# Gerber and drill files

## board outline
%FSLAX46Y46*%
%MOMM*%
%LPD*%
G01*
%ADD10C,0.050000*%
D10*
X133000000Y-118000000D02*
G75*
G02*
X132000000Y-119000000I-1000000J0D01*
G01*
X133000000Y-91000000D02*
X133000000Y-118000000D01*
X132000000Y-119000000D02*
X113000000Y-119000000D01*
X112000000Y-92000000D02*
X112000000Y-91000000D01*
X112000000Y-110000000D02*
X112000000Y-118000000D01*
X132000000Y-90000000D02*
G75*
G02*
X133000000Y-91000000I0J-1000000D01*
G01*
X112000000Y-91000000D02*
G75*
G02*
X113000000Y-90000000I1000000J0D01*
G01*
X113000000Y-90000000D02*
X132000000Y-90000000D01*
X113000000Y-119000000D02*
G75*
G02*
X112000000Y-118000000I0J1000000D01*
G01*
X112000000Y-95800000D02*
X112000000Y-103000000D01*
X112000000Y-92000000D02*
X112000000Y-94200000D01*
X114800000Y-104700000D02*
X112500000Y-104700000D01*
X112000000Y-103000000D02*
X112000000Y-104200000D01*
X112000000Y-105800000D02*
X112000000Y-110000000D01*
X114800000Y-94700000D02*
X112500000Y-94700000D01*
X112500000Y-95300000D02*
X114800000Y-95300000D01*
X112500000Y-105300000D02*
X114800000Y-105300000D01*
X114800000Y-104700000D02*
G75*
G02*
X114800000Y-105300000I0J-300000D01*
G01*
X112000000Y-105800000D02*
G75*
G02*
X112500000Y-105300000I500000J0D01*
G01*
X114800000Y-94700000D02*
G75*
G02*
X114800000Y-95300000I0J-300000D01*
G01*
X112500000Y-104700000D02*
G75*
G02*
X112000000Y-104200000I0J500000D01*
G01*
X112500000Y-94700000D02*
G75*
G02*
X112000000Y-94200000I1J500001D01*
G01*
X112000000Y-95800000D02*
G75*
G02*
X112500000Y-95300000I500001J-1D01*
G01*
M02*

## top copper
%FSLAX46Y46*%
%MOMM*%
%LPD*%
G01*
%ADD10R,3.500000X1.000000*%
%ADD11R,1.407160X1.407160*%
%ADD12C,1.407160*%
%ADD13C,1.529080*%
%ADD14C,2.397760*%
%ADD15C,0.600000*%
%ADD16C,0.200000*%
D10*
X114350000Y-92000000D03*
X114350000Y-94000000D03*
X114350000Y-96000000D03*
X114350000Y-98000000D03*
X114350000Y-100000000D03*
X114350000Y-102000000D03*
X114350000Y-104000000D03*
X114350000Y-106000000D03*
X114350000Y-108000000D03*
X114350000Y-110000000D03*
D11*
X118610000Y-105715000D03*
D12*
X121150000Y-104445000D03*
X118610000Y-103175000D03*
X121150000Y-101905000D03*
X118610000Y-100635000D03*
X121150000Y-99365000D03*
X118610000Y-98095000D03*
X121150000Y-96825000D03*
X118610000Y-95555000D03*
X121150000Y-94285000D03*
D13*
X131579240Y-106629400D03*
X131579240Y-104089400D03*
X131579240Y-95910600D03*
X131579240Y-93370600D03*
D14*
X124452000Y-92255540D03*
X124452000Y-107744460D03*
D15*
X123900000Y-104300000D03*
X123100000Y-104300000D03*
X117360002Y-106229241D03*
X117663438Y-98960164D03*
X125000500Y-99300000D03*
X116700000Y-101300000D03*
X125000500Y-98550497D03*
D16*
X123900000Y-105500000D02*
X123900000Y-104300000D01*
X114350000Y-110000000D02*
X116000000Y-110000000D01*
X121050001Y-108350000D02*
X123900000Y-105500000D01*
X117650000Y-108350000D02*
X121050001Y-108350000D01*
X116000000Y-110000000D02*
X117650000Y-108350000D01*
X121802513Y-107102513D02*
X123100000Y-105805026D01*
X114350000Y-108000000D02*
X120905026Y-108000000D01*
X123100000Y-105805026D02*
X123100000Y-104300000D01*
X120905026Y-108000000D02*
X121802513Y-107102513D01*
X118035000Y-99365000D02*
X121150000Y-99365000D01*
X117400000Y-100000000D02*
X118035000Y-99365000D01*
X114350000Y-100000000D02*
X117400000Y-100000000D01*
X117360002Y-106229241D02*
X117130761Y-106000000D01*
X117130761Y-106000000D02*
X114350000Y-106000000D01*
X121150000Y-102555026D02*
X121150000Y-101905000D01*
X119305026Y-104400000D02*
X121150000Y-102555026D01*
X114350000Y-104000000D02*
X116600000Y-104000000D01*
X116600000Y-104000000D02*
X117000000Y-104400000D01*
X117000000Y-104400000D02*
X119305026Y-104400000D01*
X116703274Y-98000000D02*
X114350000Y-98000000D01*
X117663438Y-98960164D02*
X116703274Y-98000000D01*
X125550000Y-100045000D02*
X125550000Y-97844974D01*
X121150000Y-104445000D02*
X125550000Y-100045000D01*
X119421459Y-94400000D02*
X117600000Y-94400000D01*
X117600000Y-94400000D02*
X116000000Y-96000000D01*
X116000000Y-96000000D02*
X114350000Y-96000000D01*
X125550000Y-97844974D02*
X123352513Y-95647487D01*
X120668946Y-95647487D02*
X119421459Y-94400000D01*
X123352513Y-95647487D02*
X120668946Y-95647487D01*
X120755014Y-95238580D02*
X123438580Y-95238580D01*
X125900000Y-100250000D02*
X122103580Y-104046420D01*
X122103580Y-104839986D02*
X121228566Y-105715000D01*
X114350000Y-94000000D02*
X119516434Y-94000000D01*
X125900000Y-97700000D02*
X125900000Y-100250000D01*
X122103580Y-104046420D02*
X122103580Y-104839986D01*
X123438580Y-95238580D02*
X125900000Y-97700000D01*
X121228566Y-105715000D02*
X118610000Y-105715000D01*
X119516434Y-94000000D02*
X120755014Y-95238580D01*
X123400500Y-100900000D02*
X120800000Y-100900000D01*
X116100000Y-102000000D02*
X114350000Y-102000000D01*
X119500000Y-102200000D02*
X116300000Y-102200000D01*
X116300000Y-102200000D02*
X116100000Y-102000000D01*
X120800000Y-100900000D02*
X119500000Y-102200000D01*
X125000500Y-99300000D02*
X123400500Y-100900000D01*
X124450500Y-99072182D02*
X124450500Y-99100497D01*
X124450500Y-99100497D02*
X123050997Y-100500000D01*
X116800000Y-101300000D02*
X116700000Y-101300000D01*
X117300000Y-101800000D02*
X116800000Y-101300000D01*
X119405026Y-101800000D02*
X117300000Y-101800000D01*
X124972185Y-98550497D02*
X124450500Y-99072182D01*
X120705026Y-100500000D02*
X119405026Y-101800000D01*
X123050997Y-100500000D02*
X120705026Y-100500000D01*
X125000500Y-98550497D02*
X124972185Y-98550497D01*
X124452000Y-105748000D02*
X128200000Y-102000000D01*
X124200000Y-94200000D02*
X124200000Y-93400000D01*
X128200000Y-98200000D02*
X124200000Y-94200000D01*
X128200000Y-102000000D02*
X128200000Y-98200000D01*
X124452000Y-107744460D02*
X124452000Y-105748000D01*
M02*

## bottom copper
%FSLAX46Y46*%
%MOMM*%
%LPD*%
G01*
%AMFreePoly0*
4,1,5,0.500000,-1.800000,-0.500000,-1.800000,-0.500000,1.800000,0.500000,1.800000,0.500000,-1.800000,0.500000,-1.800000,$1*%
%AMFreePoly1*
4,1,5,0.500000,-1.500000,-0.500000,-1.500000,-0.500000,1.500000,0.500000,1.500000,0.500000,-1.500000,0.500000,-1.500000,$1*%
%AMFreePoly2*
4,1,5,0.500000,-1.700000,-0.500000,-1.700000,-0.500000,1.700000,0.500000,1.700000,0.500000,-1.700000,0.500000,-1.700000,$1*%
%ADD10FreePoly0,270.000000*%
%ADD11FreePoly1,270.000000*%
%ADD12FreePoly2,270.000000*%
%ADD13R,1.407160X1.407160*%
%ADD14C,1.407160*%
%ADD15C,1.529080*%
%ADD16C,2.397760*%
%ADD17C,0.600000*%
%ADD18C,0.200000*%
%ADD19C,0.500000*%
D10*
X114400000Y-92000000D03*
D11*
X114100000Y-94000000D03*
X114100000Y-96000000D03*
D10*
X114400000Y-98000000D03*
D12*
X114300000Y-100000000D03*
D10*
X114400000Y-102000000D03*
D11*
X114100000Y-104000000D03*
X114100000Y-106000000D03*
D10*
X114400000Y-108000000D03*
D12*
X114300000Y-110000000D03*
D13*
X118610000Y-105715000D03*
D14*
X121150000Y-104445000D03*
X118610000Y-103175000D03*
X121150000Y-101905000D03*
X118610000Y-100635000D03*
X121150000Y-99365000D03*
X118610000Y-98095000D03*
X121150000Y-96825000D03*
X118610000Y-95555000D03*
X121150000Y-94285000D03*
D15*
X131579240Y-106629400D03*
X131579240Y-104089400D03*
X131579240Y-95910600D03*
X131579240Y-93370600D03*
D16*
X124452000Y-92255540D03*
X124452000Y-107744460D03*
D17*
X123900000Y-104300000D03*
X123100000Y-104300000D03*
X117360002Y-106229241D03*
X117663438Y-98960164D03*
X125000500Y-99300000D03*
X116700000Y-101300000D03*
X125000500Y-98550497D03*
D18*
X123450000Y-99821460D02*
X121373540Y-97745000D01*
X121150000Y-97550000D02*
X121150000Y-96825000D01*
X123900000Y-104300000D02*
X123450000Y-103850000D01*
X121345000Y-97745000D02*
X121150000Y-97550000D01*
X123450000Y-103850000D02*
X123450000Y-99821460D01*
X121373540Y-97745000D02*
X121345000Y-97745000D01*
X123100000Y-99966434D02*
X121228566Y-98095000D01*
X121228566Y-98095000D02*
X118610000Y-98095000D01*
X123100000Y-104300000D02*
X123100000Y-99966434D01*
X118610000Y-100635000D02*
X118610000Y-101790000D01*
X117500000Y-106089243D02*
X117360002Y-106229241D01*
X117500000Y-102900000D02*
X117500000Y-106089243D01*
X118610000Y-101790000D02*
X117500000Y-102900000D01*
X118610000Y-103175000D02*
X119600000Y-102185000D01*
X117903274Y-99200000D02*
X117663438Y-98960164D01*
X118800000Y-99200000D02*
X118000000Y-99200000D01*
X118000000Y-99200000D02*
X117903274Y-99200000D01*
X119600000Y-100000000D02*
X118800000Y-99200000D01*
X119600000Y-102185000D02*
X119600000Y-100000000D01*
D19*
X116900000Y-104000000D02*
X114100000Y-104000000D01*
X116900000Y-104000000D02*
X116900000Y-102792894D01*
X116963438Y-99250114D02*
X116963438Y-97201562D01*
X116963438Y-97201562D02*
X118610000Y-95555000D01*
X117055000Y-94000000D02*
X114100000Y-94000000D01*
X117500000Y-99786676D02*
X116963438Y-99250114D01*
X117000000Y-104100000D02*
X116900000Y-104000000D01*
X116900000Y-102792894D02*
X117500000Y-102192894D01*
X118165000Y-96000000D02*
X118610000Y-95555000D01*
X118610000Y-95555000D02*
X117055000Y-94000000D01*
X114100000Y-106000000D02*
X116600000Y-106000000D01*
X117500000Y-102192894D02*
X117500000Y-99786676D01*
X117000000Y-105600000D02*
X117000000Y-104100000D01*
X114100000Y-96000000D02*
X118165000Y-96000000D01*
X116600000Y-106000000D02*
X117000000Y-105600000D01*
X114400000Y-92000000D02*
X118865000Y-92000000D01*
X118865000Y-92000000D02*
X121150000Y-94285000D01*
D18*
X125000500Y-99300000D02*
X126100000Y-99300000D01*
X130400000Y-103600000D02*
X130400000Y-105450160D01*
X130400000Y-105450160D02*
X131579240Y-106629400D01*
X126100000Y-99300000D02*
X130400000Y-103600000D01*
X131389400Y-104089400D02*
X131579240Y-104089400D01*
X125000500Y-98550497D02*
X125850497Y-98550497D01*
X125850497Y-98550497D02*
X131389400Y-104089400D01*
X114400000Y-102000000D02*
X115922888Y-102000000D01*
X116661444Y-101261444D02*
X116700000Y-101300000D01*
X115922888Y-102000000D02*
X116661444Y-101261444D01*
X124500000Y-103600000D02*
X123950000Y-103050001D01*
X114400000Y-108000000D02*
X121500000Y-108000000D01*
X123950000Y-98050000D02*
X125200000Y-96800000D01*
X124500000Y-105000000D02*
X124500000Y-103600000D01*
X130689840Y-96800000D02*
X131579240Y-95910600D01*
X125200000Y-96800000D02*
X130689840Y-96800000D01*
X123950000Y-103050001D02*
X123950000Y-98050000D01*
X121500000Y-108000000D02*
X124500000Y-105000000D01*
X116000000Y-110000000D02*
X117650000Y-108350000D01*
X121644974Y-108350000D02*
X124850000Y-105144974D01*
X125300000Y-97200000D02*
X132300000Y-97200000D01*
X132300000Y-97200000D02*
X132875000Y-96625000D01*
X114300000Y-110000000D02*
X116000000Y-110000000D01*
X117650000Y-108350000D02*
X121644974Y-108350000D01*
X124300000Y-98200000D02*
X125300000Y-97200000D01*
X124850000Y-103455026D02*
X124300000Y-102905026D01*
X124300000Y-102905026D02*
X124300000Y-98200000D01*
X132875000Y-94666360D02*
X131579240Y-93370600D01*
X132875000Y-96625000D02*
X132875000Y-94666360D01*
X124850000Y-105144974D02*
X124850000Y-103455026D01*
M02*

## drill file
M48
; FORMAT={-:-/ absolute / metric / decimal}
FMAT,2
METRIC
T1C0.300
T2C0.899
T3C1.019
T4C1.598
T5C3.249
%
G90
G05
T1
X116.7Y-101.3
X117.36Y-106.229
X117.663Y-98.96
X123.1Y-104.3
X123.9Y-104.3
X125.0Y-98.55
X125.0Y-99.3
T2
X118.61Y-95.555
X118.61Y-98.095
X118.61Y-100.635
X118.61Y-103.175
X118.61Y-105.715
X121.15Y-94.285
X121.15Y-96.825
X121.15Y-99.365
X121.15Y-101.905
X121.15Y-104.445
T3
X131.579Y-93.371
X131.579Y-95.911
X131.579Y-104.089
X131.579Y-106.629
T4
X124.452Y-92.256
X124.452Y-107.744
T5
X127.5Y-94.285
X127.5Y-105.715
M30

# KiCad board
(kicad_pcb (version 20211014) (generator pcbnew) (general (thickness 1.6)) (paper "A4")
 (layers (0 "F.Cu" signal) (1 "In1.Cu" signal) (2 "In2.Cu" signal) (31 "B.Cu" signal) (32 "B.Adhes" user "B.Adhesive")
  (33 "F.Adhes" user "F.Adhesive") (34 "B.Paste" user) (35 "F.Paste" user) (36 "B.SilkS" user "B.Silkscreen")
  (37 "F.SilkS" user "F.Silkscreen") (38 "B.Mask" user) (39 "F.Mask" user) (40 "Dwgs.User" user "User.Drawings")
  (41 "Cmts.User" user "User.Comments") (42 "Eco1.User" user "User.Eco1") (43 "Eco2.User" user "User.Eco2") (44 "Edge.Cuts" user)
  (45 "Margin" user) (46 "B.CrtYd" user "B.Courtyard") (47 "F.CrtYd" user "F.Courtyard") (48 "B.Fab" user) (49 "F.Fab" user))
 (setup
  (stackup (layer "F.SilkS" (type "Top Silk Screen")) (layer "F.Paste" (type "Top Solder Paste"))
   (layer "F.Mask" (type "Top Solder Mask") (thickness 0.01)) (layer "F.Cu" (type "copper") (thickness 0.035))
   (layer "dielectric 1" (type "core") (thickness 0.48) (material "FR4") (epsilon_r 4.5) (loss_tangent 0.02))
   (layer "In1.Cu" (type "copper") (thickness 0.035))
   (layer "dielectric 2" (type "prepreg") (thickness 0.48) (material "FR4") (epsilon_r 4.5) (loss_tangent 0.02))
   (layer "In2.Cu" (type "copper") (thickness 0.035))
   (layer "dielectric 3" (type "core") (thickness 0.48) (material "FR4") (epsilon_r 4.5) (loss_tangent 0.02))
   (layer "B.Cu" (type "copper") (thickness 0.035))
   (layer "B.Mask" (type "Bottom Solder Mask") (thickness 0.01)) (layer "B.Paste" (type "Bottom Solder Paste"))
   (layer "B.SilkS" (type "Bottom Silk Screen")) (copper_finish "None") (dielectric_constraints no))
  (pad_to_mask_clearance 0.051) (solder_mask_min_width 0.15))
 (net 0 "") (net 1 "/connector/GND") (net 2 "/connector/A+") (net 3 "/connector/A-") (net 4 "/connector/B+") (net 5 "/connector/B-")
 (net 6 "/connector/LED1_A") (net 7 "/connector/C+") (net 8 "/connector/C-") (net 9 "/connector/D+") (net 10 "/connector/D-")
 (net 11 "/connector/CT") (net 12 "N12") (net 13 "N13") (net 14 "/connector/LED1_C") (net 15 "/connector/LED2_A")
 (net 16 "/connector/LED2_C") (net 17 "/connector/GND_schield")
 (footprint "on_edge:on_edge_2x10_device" (layer "F.Cu") (at 112 96 -90)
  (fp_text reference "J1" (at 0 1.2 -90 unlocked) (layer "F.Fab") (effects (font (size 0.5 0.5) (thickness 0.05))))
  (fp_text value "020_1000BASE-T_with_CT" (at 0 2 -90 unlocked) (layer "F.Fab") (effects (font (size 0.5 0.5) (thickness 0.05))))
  (fp_line (start -0.2 0) (end 7 0) (layer "Edge.Cuts") (width 0.05))
  (fp_line (start -4 0) (end -1.8 0) (layer "Edge.Cuts") (width 0.05))
  (fp_line (start 8.7 -2.8) (end 8.7 -0.5) (layer "Edge.Cuts") (width 0.05))
  (fp_line (start 7 0) (end 8.2 0) (layer "Edge.Cuts") (width 0.05))
  (fp_line (start 9.8 0) (end 14 0) (layer "Edge.Cuts") (width 0.05))
  (fp_line (start -1.3 -2.8) (end -1.3 -0.5) (layer "Edge.Cuts") (width 0.05))
  (fp_line (start -0.7 -0.5) (end -0.7 -2.8) (layer "Edge.Cuts") (width 0.05))
  (fp_line (start 9.3 -0.5) (end 9.3 -2.8) (layer "Edge.Cuts") (width 0.05))
  (fp_arc (start 8.7 -2.8) (mid 9 -3.1) (end 9.3 -2.8) (layer "Edge.Cuts") (width 0.05))
  (fp_arc (start 9.8 0) (mid 9.446447 -0.146447) (end 9.3 -0.5) (layer "Edge.Cuts") (width 0.05))
  (fp_arc (start -1.3 -2.8) (mid -1 -3.1) (end -0.7 -2.8) (layer "Edge.Cuts") (width 0.05))
  (fp_arc (start 8.7 -0.5) (mid 8.553553 -0.146447) (end 8.2 0) (layer "Edge.Cuts") (width 0.05))
  (fp_arc (start -1.3 -0.5) (mid -1.446447 -0.146447) (end -1.8 0) (layer "Edge.Cuts") (width 0.05))
  (fp_arc (start -0.2 0) (mid -0.553553 -0.146447) (end -0.7 -0.5) (layer "Edge.Cuts") (width 0.05))
  (pad "1" smd rect (at -4 -2.35 90) (size 1 3.5) (layers "F.Cu" "F.Mask") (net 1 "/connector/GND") (zone_connect 0))
  (pad "2" smd rect (at -2 -2.35 270) (size 1 3.5) (layers "F.Cu" "F.Mask") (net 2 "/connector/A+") (zone_connect 0))
  (pad "3" smd rect (at 0 -2.35 270) (size 1 3.5) (layers "F.Cu" "F.Mask") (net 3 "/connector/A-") (zone_connect 0))
  (pad "4" smd rect (at 2 -2.35 90) (size 1 3.5) (layers "F.Cu" "F.Mask") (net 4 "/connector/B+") (zone_connect 0))
  (pad "5" smd rect (at 4 -2.35 90) (size 1 3.5) (layers "F.Cu" "F.Mask") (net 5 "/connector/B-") (zone_connect 0))
  (pad "6" smd rect (at 6 -2.35 90) (size 1 3.5) (layers "F.Cu" "F.Mask") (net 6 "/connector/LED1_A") (zone_connect 0))
  (pad "7" smd rect (at 8 -2.35 270) (size 1 3.5) (layers "F.Cu" "F.Mask") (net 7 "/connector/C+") (zone_connect 0))
  (pad "8" smd rect (at 10 -2.35 270) (size 1 3.5) (layers "F.Cu" "F.Mask") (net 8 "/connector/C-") (zone_connect 0))
  (pad "9" smd rect (at 12 -2.35 90) (size 1 3.5) (layers "F.Cu" "F.Mask") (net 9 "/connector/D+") (zone_connect 0))
  (pad "10" smd rect (at 14 -2.35 90) (size 1 3.5) (layers "F.Cu" "F.Mask") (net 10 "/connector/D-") (zone_connect 0))
  (pad "11" smd custom (at -4 -2.4 270) (size 1 3.6) (layers "B.Cu" "B.Mask") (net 1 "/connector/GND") (zone_connect 0)
   (options (clearance outline) (anchor rect)) (primitives))
  (pad "12" smd custom (at -2 -2.1 270) (size 1 3) (layers "B.Cu" "B.Mask") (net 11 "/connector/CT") (zone_connect 0)
   (options (clearance outline) (anchor rect)) (primitives))
  (pad "13" smd custom (at 0 -2.1 270) (size 1 3) (layers "B.Cu" "B.Mask") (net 11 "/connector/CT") (zone_connect 0)
   (options (clearance outline) (anchor rect)) (primitives))
  (pad "14" smd custom (at 2 -2.4 270) (size 1 3.6) (layers "B.Cu" "B.Mask") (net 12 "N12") (zone_connect 0)
   (options (clearance outline) (anchor rect)) (primitives))
  (pad "15" smd custom (at 4 -2.3 270) (size 1 3.4) (layers "B.Cu" "B.Mask") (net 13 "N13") (zone_connect 0)
   (options (clearance outline) (anchor rect)) (primitives))
  (pad "16" smd custom (at 6 -2.4 270) (size 1 3.6) (layers "B.Cu" "B.Mask") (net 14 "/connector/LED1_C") (zone_connect 0)
   (options (clearance outline) (anchor rect)) (primitives))
  (pad "17" smd custom (at 8 -2.1 270) (size 1 3) (layers "B.Cu" "B.Mask") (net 11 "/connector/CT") (zone_connect 0)
   (options (clearance outline) (anchor rect)) (primitives))
  (pad "18" smd custom (at 10 -2.1 270) (size 1 3) (layers "B.Cu" "B.Mask") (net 11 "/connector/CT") (zone_connect 0)
   (options (clearance outline) (anchor rect)) (primitives))
  (pad "19" smd custom (at 12 -2.4 270) (size 1 3.6) (layers "B.Cu" "B.Mask") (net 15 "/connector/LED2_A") (zone_connect 0)
   (options (clearance outline) (anchor rect)) (primitives))
  (pad "20" smd custom (at 14 -2.3 270) (size 1 3.4) (layers "B.Cu" "B.Mask") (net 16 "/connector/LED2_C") (zone_connect 0)
   (options (clearance outline) (anchor rect)) (primitives))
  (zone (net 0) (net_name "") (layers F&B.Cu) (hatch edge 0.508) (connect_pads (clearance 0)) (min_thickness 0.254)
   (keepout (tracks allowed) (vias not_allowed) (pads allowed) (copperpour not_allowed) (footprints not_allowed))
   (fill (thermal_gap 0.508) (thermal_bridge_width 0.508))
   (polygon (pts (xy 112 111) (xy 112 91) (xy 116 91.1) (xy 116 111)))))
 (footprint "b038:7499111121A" (layer "F.Cu") (at 127.5 100 -90)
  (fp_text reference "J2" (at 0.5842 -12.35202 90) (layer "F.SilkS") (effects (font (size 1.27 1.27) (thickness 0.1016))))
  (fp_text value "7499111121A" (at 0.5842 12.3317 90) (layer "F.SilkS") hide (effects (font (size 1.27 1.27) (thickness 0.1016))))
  (pad "" np_thru_hole circle (at 5.715 0 270) (size 3.24866 3.24866) (drill 3.24866) (layers *.Cu *.Mask))
  (pad "" np_thru_hole circle (at -5.715 0 270) (size 3.24866 3.24866) (drill 3.24866) (layers *.Cu *.Mask))
  (pad "1" thru_hole rect (at 5.715 8.89 270) (size 1.40716 1.40716) (drill 0.89916) (layers *.Cu *.Paste *.Mask) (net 2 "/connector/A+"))
  (pad "2" thru_hole circle (at 4.445 6.35 270) (size 1.40716 1.40716) (drill 0.89916) (layers *.Cu *.Paste *.Mask) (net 3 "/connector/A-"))
  (pad "3" thru_hole circle (at 3.175 8.89 270) (size 1.40716 1.40716) (drill 0.89916) (layers *.Cu *.Paste *.Mask) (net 4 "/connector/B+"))
  (pad "4" thru_hole circle (at 1.905 6.35 270) (size 1.40716 1.40716) (drill 0.89916) (layers *.Cu *.Paste *.Mask) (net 7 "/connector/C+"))
  (pad "5" thru_hole circle (at 0.635 8.89 270) (size 1.40716 1.40716) (drill 0.89916) (layers *.Cu *.Paste *.Mask) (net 8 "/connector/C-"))
  (pad "6" thru_hole circle (at -0.635 6.35 270) (size 1.40716 1.40716) (drill 0.89916) (layers *.Cu *.Paste *.Mask) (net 5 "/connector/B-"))
  (pad "7" thru_hole circle (at -1.905 8.89 270) (size 1.40716 1.40716) (drill 0.89916) (layers *.Cu *.Paste *.Mask) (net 9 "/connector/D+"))
  (pad "8" thru_hole circle (at -3.175 6.35 270) (size 1.40716 1.40716) (drill 0.89916) (layers *.Cu *.Paste *.Mask)
   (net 10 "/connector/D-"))
  (pad "9" thru_hole circle (at -4.445 8.89 270) (size 1.40716 1.40716) (drill 0.89916) (layers *.Cu *.Paste *.Mask)
   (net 11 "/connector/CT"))
  (pad "10" thru_hole circle (at -5.715 6.35 270) (size 1.40716 1.40716) (drill 0.89916) (layers *.Cu *.Paste *.Mask)
   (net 1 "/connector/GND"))
  (pad "11" thru_hole circle (at 6.6294 -4.07924 270) (size 1.52908 1.52908) (drill 1.01854) (layers *.Cu *.Paste *.Mask)
   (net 6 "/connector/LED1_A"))
  (pad "12" thru_hole circle (at 4.0894 -4.07924 270) (size 1.52908 1.52908) (drill 1.01854) (layers *.Cu *.Paste *.Mask)
   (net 14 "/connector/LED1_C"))
  (pad "13" thru_hole circle (at -4.0894 -4.07924 270) (size 1.52908 1.52908) (drill 1.01854) (layers *.Cu *.Paste *.Mask)
   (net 15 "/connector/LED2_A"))
  (pad "14" thru_hole circle (at -6.6294 -4.07924 270) (size 1.52908 1.52908) (drill 1.01854) (layers *.Cu *.Paste *.Mask)
   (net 16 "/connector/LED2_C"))
  (pad "Z1" thru_hole circle (at -7.74446 3.048 270) (size 2.39776 2.39776) (drill 1.59766) (layers *.Cu *.Paste *.Mask)
   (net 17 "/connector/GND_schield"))
  (pad "Z2" thru_hole circle (at 7.74446 3.048 270) (size 2.39776 2.39776) (drill 1.59766) (layers *.Cu *.Paste *.Mask)
   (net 17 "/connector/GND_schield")))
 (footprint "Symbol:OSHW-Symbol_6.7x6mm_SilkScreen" (layer "F.Cu") (at 129.45 113.2)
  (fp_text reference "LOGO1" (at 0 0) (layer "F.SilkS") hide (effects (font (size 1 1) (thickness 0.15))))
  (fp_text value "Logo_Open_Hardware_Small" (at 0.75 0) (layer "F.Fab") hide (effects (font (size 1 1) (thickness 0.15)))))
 (gr_arc (start 133 118) (mid 132.707107 118.707107) (end 132 119) (layer "Edge.Cuts") (width 0.05))
 (gr_line (start 133 91) (end 133 118) (layer "Edge.Cuts") (width 0.05))
 (gr_line (start 132 119) (end 113 119) (layer "Edge.Cuts") (width 0.05))
 (gr_line (start 112 92) (end 112 91) (layer "Edge.Cuts") (width 0.05))
 (gr_line (start 112 110) (end 112 118) (layer "Edge.Cuts") (width 0.05))
 (gr_arc (start 132 90) (mid 132.707107 90.292893) (end 133 91) (layer "Edge.Cuts") (width 0.05))
 (gr_arc (start 112 91) (mid 112.292893 90.292893) (end 113 90) (layer "Edge.Cuts") (width 0.05))
 (gr_line (start 113 90) (end 132 90) (layer "Edge.Cuts") (width 0.05))
 (gr_arc (start 113 119) (mid 112.292893 118.707107) (end 112 118) (layer "Edge.Cuts") (width 0.05))
 (segment (start 123.9 105.5) (end 123.9 104.3) (width 0.2) (layer "F.Cu") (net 10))
 (segment (start 114.35 110) (end 116 110) (width 0.2) (layer "F.Cu") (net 10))
 (segment (start 121.050001 108.35) (end 123.9 105.5) (width 0.2) (layer "F.Cu") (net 10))
 (segment (start 117.65 108.35) (end 121.050001 108.35) (width 0.2) (layer "F.Cu") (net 10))
 (segment (start 116 110) (end 117.65 108.35) (width 0.2) (layer "F.Cu") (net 10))
 (via (at 123.9 104.3) (size 0.6) (drill 0.3) (layers "F.Cu" "B.Cu") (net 10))
 (segment (start 123.45 99.82146) (end 121.37354 97.745) (width 0.2) (layer "B.Cu") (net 10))
 (segment (start 121.15 97.55) (end 121.15 96.825) (width 0.2) (layer "B.Cu") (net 10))
 (segment (start 123.9 104.3) (end 123.45 103.85) (width 0.2) (layer "B.Cu") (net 10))
 (segment (start 121.345 97.745) (end 121.15 97.55) (width 0.2) (layer "B.Cu") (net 10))
 (segment (start 123.45 103.85) (end 123.45 99.82146) (width 0.2) (layer "B.Cu") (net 10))
 (segment (start 121.37354 97.745) (end 121.345 97.745) (width 0.2) (layer "B.Cu") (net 10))
 (segment (start 121.802513 107.102513) (end 123.1 105.805026) (width 0.2) (layer "F.Cu") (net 9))
 (segment (start 114.35 108) (end 120.905026 108) (width 0.2) (layer "F.Cu") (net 9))
 (segment (start 123.1 105.805026) (end 123.1 104.3) (width 0.2) (layer "F.Cu") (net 9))
 (segment (start 120.905026 108) (end 121.802513 107.102513) (width 0.2) (layer "F.Cu") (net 9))
 (via (at 123.1 104.3) (size 0.6) (drill 0.3) (layers "F.Cu" "B.Cu") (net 9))
 (segment (start 123.1 99.966434) (end 121.228566 98.095) (width 0.2) (layer "B.Cu") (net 9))
 (segment (start 121.228566 98.095) (end 118.61 98.095) (width 0.2) (layer "B.Cu") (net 9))
 (segment (start 123.1 104.3) (end 123.1 99.966434) (width 0.2) (layer "B.Cu") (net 9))
 (segment (start 118.035 99.365) (end 121.15 99.365) (width 0.2) (layer "F.Cu") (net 5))
 (segment (start 117.4 100) (end 118.035 99.365) (width 0.2) (layer "F.Cu") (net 5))
 (segment (start 114.35 100) (end 117.4 100) (width 0.2) (layer "F.Cu") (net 5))
 (segment (start 117.360002 106.229241) (end 117.130761 106) (width 0.2) (layer "F.Cu") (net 8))
 (segment (start 117.130761 106) (end 114.35 106) (width 0.2) (layer "F.Cu") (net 8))
 (via (at 117.360002 106.229241) (size 0.6) (drill 0.3) (layers "F.Cu" "B.Cu") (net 8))
 (segment (start 118.61 100.635) (end 118.61 101.79) (width 0.2) (layer "B.Cu") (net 8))
 (segment (start 117.5 106.089243) (end 117.360002 106.229241) (width 0.2) (layer "B.Cu") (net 8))
 (segment (start 117.5 102.9) (end 117.5 106.089243) (width 0.2) (layer "B.Cu") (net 8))
 (segment (start 118.61 101.79) (end 117.5 102.9) (width 0.2) (layer "B.Cu") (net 8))
 (segment (start 121.15 102.555026) (end 121.15 101.905) (width 0.2) (layer "F.Cu") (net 7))
 (segment (start 119.305026 104.4) (end 121.15 102.555026) (width 0.2) (layer "F.Cu") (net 7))
 (segment (start 114.35 104) (end 116.6 104) (width 0.2) (layer "F.Cu") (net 7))
 (segment (start 116.6 104) (end 117 104.4) (width 0.2) (layer "F.Cu") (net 7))
 (segment (start 117 104.4) (end 119.305026 104.4) (width 0.2) (layer "F.Cu") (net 7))
 (segment (start 116.703274 98) (end 114.35 98) (width 0.2) (layer "F.Cu") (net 4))
 (segment (start 117.663438 98.960164) (end 116.703274 98) (width 0.2) (layer "F.Cu") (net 4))
 (via (at 117.663438 98.960164) (size 0.6) (drill 0.3) (layers "F.Cu" "B.Cu") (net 4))
 (segment (start 118.61 103.175) (end 119.6 102.185) (width 0.2) (layer "B.Cu") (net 4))
 (segment (start 117.903274 99.2) (end 117.663438 98.960164) (width 0.2) (layer "B.Cu") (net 4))
 (segment (start 118.8 99.2) (end 118 99.2) (width 0.2) (layer "B.Cu") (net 4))
 (segment (start 118 99.2) (end 117.903274 99.2) (width 0.2) (layer "B.Cu") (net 4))
 (segment (start 119.6 100) (end 118.8 99.2) (width 0.2) (layer "B.Cu") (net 4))
 (segment (start 119.6 102.185) (end 119.6 100) (width 0.2) (layer "B.Cu") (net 4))
 (segment (start 125.55 100.045) (end 125.55 97.844974) (width 0.2) (layer "F.Cu") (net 3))
 (segment (start 121.15 104.445) (end 125.55 100.045) (width 0.2) (layer "F.Cu") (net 3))
 (segment (start 119.421459 94.4) (end 117.6 94.4) (width 0.2) (layer "F.Cu") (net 3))
 (segment (start 117.6 94.4) (end 116 96) (width 0.2) (layer "F.Cu") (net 3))
 (segment (start 116 96) (end 114.35 96) (width 0.2) (layer "F.Cu") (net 3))
 (segment (start 125.55 97.844974) (end 123.352513 95.647487) (width 0.2) (layer "F.Cu") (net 3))
 (segment (start 120.668946 95.647487) (end 119.421459 94.4) (width 0.2) (layer "F.Cu") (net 3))
 (segment (start 123.352513 95.647487) (end 120.668946 95.647487) (width 0.2) (layer "F.Cu") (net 3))
 (segment (start 120.755014 95.23858) (end 123.43858 95.23858) (width 0.2) (layer "F.Cu") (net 2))
 (segment (start 125.9 100.25) (end 122.10358 104.04642) (width 0.2) (layer "F.Cu") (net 2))
 (segment (start 122.10358 104.839986) (end 121.228566 105.715) (width 0.2) (layer "F.Cu") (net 2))
 (segment (start 114.35 94) (end 119.516434 94) (width 0.2) (layer "F.Cu") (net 2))
 (segment (start 125.9 97.7) (end 125.9 100.25) (width 0.2) (layer "F.Cu") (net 2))
 (segment (start 122.10358 104.04642) (end 122.10358 104.839986) (width 0.2) (layer "F.Cu") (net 2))
 (segment (start 123.43858 95.23858) (end 125.9 97.7) (width 0.2) (layer "F.Cu") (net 2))
 (segment (start 121.228566 105.715) (end 118.61 105.715) (width 0.2) (layer "F.Cu") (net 2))
 (segment (start 119.516434 94) (end 120.755014 95.23858) (width 0.2) (layer "F.Cu") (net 2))
 (segment (start 116.9 104) (end 114.1 104) (width 0.5) (layer "B.Cu") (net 11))
 (segment (start 116.9 104) (end 116.9 102.792894) (width 0.5) (layer "B.Cu") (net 11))
 (segment (start 116.963438 99.250114) (end 116.963438 97.201562) (width 0.5) (layer "B.Cu") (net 11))
 (segment (start 116.963438 97.201562) (end 118.61 95.555) (width 0.5) (layer "B.Cu") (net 11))
 (segment (start 117.055 94) (end 114.1 94) (width 0.5) (layer "B.Cu") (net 11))
 (segment (start 117.5 99.786676) (end 116.963438 99.250114) (width 0.5) (layer "B.Cu") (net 11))
 (segment (start 117 104.1) (end 116.9 104) (width 0.5) (layer "B.Cu") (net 11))
 (segment (start 116.9 102.792894) (end 117.5 102.192894) (width 0.5) (layer "B.Cu") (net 11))
 (segment (start 118.165 96) (end 118.61 95.555) (width 0.5) (layer "B.Cu") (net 11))
 (segment (start 118.61 95.555) (end 117.055 94) (width 0.5) (layer "B.Cu") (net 11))
 (segment (start 114.1 106) (end 116.6 106) (width 0.5) (layer "B.Cu") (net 11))
 (segment (start 117.5 102.192894) (end 117.5 99.786676) (width 0.5) (layer "B.Cu") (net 11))
 (segment (start 117 105.6) (end 117 104.1) (width 0.5) (layer "B.Cu") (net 11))
 (segment (start 114.1 96) (end 118.165 96) (width 0.5) (layer "B.Cu") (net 11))
 (segment (start 116.6 106) (end 117 105.6) (width 0.5) (layer "B.Cu") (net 11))
 (segment (start 114.4 92) (end 118.865 92) (width 0.5) (layer "B.Cu") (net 1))
 (segment (start 118.865 92) (end 121.15 94.285) (width 0.5) (layer "B.Cu") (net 1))
 (segment (start 123.4005 100.9) (end 120.8 100.9) (width 0.2) (layer "F.Cu") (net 6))
 (segment (start 116.1 102) (end 114.35 102) (width 0.2) (layer "F.Cu") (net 6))
 (segment (start 119.5 102.2) (end 116.3 102.2) (width 0.2) (layer "F.Cu") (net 6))
 (segment (start 116.3 102.2) (end 116.1 102) (width 0.2) (layer "F.Cu") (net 6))
 (segment (start 120.8 100.9) (end 119.5 102.2) (width 0.2) (layer "F.Cu") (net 6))
 (segment (start 125.0005 99.3) (end 123.4005 100.9) (width 0.2) (layer "F.Cu") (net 6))
 (via (at 125.0005 99.3) (size 0.6) (drill 0.3) (layers "F.Cu" "B.Cu") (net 6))
 (segment (start 125.0005 99.3) (end 126.1 99.3) (width 0.2) (layer "B.Cu") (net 6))
 (segment (start 130.4 103.6) (end 130.4 105.45016) (width 0.2) (layer "B.Cu") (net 6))
 (segment (start 130.4 105.45016) (end 131.57924 106.6294) (width 0.2) (layer "B.Cu") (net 6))
 (segment (start 126.1 99.3) (end 130.4 103.6) (width 0.2) (layer "B.Cu") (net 6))
 (segment (start 124.4505 99.072182) (end 124.4505 99.100497) (width 0.2) (layer "F.Cu") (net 14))
 (segment (start 124.4505 99.100497) (end 123.050997 100.5) (width 0.2) (layer "F.Cu") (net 14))
 (segment (start 116.8 101.3) (end 116.7 101.3) (width 0.2) (layer "F.Cu") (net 14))
 (segment (start 117.3 101.8) (end 116.8 101.3) (width 0.2) (layer "F.Cu") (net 14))
 (segment (start 119.405026 101.8) (end 117.3 101.8) (width 0.2) (layer "F.Cu") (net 14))
 (segment (start 124.972185 98.550497) (end 124.4505 99.072182) (width 0.2) (layer "F.Cu") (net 14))
 (segment (start 120.705026 100.5) (end 119.405026 101.8) (width 0.2) (layer "F.Cu") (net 14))
 (segment (start 123.050997 100.5) (end 120.705026 100.5) (width 0.2) (layer "F.Cu") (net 14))
 (segment (start 125.0005 98.550497) (end 124.972185 98.550497) (width 0.2) (layer "F.Cu") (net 14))
 (via (at 116.7 101.3) (size 0.6) (drill 0.3) (layers "F.Cu" "B.Cu") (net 14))
 (via (at 125.0005 98.550497) (size 0.6) (drill 0.3) (layers "F.Cu" "B.Cu") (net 14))
 (segment (start 131.3894 104.0894) (end 131.57924 104.0894) (width 0.2) (layer "B.Cu") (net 14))
 (segment (start 125.0005 98.550497) (end 125.850497 98.550497) (width 0.2) (layer "B.Cu") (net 14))
 (segment (start 125.850497 98.550497) (end 131.3894 104.0894) (width 0.2) (layer "B.Cu") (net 14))
 (segment (start 114.4 102) (end 115.922888 102) (width 0.2) (layer "B.Cu") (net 14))
 (segment (start 116.661444 101.261444) (end 116.7 101.3) (width 0.2) (layer "B.Cu") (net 14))
 (segment (start 115.922888 102) (end 116.661444 101.261444) (width 0.2) (layer "B.Cu") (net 14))
 (segment (start 124.5 103.6) (end 123.95 103.050001) (width 0.2) (layer "B.Cu") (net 15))
 (segment (start 114.4 108) (end 121.5 108) (width 0.2) (layer "B.Cu") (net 15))
 (segment (start 123.95 98.05) (end 125.2 96.8) (width 0.2) (layer "B.Cu") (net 15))
 (segment (start 124.5 105) (end 124.5 103.6) (width 0.2) (layer "B.Cu") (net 15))
 (segment (start 130.68984 96.8) (end 131.57924 95.9106) (width 0.2) (layer "B.Cu") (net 15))
 (segment (start 125.2 96.8) (end 130.68984 96.8) (width 0.2) (layer "B.Cu") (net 15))
 (segment (start 123.95 103.050001) (end 123.95 98.05) (width 0.2) (layer "B.Cu") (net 15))
 (segment (start 121.5 108) (end 124.5 105) (width 0.2) (layer "B.Cu") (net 15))
 (segment (start 116 110) (end 117.65 108.35) (width 0.2) (layer "B.Cu") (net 16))
 (segment (start 121.644974 108.35) (end 124.85 105.144974) (width 0.2) (layer "B.Cu") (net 16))
 (segment (start 125.3 97.2) (end 132.3 97.2) (width 0.2) (layer "B.Cu") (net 16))
 (segment (start 132.3 97.2) (end 132.875 96.625) (width 0.2) (layer "B.Cu") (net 16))
 (segment (start 114.3 110) (end 116 110) (width 0.2) (layer "B.Cu") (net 16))
 (segment (start 117.65 108.35) (end 121.644974 108.35) (width 0.2) (layer "B.Cu") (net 16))
 (segment (start 124.3 98.2) (end 125.3 97.2) (width 0.2) (layer "B.Cu") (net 16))
 (segment (start 124.85 103.455026) (end 124.3 102.905026) (width 0.2) (layer "B.Cu") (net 16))
 (segment (start 124.3 102.905026) (end 124.3 98.2) (width 0.2) (layer "B.Cu") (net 16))
 (segment (start 132.875 94.66636) (end 131.57924 93.3706) (width 0.2) (layer "B.Cu") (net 16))
 (segment (start 132.875 96.625) (end 132.875 94.66636) (width 0.2) (layer "B.Cu") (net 16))
 (segment (start 124.85 105.144974) (end 124.85 103.455026) (width 0.2) (layer "B.Cu") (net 16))
 (segment (start 124.452 105.748) (end 128.2 102) (width 0.2) (layer "F.Cu") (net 17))
 (segment (start 124.2 94.2) (end 124.2 93.4) (width 0.2) (layer "F.Cu") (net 17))
 (segment (start 128.2 98.2) (end 124.2 94.2) (width 0.2) (layer "F.Cu") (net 17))
 (segment (start 128.2 102) (end 128.2 98.2) (width 0.2) (layer "F.Cu") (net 17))
 (segment (start 124.452 107.74446) (end 124.452 105.748) (width 0.2) (layer "F.Cu") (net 17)))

